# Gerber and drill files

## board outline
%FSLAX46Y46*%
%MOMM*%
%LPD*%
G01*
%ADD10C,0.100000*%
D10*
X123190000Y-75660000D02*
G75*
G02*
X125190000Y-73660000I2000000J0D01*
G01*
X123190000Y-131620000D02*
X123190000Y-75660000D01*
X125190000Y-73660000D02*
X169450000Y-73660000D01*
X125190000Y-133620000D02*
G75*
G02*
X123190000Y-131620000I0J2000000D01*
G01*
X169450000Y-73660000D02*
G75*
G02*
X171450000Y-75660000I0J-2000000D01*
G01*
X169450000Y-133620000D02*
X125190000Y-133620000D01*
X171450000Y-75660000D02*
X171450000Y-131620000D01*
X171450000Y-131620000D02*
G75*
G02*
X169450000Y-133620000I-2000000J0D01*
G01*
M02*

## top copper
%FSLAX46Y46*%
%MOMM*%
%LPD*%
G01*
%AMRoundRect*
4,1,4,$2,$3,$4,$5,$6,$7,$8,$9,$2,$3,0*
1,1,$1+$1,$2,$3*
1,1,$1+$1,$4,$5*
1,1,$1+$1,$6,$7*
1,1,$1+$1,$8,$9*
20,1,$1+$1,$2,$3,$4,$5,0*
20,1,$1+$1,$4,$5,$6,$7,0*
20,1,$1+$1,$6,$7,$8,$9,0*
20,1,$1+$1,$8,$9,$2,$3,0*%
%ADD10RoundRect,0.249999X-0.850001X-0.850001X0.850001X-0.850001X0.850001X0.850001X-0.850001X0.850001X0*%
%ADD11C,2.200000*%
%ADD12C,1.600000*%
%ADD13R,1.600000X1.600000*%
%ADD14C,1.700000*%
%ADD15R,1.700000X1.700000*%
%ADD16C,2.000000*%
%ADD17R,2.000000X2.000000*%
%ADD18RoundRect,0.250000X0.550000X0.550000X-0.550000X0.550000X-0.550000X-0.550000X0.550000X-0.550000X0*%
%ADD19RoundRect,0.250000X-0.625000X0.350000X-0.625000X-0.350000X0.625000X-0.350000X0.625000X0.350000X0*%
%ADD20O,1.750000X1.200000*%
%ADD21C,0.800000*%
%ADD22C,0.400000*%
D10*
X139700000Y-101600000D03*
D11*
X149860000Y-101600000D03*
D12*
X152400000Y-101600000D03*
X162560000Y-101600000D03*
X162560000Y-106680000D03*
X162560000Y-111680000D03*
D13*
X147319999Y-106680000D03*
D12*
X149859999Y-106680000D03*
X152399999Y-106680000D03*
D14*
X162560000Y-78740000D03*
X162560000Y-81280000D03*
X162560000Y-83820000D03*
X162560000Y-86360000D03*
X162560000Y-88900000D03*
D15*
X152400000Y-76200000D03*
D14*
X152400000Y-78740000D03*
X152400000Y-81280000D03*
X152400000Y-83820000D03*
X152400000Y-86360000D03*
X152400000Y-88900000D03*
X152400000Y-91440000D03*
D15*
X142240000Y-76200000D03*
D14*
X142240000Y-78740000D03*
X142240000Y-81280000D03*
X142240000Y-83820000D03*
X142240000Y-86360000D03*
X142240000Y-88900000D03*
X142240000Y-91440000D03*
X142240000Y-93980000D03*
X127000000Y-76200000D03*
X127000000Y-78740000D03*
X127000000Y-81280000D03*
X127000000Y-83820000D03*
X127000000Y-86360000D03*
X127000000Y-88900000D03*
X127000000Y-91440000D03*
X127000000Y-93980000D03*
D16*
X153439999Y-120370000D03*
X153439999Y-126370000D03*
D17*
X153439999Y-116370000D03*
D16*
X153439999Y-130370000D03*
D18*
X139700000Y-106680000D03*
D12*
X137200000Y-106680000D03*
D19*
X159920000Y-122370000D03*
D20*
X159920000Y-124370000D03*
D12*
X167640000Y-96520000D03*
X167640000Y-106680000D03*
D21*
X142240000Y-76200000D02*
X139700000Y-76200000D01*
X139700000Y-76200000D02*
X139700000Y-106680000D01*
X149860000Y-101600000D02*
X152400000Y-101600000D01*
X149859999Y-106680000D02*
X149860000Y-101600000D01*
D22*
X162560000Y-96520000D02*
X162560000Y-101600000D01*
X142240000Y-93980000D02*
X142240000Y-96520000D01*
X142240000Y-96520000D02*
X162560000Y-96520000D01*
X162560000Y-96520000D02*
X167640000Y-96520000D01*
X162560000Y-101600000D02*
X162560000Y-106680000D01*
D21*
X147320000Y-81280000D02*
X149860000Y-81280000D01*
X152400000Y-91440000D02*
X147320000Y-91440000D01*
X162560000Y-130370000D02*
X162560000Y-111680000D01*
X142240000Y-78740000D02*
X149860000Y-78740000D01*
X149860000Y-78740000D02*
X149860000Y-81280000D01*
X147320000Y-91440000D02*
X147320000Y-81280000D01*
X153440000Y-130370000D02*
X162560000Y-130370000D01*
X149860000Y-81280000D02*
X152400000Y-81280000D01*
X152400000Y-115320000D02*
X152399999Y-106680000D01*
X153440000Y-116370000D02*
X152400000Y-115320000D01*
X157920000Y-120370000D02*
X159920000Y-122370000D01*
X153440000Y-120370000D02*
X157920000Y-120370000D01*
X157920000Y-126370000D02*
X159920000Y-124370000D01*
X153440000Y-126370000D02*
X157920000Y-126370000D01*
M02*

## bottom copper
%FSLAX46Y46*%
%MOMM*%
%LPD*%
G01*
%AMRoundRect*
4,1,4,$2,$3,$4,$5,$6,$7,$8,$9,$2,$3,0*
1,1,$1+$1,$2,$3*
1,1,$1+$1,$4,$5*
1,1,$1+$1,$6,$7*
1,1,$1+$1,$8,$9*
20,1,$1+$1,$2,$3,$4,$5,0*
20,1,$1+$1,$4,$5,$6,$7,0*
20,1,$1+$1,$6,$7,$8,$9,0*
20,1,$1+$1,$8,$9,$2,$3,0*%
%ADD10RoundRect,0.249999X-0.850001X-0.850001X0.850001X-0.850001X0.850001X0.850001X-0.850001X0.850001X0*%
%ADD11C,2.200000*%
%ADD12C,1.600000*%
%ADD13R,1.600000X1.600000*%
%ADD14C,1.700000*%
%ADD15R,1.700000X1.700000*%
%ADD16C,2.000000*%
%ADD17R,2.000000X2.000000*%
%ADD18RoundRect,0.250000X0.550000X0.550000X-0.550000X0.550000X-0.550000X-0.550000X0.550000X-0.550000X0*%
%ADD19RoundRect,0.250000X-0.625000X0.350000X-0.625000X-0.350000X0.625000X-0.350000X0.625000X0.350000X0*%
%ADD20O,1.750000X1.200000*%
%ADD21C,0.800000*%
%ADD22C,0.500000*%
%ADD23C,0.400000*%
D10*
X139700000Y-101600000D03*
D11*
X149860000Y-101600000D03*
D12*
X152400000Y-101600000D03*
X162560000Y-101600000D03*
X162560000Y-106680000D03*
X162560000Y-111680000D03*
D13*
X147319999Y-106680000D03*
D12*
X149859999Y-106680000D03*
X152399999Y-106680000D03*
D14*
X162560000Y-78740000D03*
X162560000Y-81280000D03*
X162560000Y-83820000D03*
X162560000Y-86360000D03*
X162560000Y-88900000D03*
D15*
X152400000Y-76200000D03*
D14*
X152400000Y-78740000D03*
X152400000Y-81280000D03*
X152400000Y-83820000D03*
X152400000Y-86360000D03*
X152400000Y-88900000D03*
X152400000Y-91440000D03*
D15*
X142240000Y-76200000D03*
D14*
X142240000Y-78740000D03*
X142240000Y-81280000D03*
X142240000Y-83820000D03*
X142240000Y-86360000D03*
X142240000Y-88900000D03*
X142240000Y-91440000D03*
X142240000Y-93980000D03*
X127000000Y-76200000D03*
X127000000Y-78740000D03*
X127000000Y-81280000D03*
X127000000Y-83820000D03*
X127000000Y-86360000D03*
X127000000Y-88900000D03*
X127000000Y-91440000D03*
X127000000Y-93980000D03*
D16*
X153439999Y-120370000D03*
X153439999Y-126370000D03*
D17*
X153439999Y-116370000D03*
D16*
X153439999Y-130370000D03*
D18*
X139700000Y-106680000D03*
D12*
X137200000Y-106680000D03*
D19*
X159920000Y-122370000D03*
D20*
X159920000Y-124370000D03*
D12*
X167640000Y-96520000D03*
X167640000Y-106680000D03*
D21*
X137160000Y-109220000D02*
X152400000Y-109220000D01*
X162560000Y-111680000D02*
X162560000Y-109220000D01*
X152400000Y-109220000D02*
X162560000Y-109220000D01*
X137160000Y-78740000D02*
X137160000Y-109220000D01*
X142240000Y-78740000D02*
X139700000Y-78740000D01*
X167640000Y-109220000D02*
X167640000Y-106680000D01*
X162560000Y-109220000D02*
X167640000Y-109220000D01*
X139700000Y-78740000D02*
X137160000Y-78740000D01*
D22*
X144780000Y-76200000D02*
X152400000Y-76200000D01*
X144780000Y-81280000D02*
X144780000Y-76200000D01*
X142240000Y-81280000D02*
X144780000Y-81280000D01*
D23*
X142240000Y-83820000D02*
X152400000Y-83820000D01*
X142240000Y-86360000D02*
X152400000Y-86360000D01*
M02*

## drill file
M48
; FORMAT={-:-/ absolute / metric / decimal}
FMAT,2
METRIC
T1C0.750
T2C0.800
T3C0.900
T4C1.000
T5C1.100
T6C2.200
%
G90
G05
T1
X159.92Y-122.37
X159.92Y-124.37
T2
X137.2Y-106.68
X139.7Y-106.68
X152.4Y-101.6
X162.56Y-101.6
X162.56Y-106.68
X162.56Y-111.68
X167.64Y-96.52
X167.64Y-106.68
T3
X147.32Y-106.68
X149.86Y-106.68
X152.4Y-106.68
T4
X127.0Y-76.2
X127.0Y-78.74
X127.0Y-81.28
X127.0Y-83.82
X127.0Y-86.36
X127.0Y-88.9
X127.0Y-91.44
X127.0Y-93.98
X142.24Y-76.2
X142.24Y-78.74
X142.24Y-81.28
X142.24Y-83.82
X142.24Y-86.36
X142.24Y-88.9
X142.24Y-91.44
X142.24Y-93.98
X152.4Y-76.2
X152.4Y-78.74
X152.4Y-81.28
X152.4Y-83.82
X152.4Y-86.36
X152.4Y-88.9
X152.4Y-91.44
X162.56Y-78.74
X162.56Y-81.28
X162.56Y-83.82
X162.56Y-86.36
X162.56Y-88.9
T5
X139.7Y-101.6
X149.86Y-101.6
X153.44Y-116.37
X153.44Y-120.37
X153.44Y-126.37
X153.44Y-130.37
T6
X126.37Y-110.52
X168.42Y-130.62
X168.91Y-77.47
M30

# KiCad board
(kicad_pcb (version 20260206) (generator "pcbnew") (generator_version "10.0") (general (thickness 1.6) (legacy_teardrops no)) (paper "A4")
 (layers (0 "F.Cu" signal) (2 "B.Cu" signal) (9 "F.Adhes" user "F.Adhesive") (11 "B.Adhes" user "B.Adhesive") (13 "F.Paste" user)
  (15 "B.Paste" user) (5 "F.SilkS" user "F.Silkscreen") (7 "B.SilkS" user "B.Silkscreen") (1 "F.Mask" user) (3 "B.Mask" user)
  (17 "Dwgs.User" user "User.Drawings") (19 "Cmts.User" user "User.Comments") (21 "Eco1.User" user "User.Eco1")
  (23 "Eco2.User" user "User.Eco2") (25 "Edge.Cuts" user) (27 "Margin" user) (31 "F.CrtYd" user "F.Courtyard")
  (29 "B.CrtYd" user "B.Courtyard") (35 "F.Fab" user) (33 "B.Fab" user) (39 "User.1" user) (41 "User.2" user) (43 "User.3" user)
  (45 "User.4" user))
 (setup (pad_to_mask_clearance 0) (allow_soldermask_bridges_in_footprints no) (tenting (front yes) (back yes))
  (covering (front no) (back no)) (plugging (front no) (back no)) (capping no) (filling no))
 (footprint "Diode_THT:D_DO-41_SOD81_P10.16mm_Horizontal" (layer "F.Cu") (at 139.7 101.6)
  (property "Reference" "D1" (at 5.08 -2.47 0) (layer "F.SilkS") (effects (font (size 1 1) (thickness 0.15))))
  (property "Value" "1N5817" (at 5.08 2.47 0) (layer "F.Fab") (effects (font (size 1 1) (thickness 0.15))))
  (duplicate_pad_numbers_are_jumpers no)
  (pad "1" thru_hole roundrect (at 0 0) (size 2.2 2.2) (drill 1.1) (layers "*.Cu" "*.Mask") (remove_unused_layers no)
   (roundrect_rratio 0.113636) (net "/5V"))
  (pad "2" thru_hole circle (at 10.16 0) (size 2.2 2.2) (drill 1.1) (layers "*.Cu" "*.Mask") (remove_unused_layers no) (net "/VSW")))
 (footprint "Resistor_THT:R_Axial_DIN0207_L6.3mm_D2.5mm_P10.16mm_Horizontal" (layer "F.Cu") (at 152.4 101.6)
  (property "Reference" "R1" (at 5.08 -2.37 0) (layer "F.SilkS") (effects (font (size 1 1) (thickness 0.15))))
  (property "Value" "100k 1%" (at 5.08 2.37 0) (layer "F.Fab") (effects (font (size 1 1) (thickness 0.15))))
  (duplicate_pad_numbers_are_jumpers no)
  (pad "1" thru_hole circle (at 0 0) (size 1.6 1.6) (drill 0.8) (layers "*.Cu" "*.Mask") (remove_unused_layers no) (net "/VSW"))
  (pad "2" thru_hole circle (at 10.16 0) (size 1.6 1.6) (drill 0.8) (layers "*.Cu" "*.Mask") (remove_unused_layers no) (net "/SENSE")))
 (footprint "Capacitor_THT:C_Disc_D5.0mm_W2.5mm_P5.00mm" (layer "F.Cu") (at 162.56 106.68 -90)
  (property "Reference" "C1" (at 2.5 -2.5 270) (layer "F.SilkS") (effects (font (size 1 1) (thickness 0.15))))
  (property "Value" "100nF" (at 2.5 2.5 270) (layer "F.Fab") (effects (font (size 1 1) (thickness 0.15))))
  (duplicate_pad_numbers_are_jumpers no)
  (pad "1" thru_hole circle (at 0 0 270) (size 1.6 1.6) (drill 0.8) (layers "*.Cu" "*.Mask") (remove_unused_layers no) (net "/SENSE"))
  (pad "2" thru_hole circle (at 5 0 270) (size 1.6 1.6) (drill 0.8) (layers "*.Cu" "*.Mask") (remove_unused_layers no) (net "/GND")))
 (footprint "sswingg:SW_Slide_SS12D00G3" (layer "F.Cu") (at 149.859999 106.68)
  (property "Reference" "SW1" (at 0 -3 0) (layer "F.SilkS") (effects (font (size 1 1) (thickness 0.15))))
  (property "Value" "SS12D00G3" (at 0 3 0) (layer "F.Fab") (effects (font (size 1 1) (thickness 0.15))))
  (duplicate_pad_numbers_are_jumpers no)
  (pad "1" thru_hole rect (at -2.54 0) (size 1.6 1.6) (drill 0.9) (layers "*.Cu" "*.Mask") (remove_unused_layers no)
   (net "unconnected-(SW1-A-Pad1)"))
  (pad "2" thru_hole circle (at 0 0) (size 1.6 1.6) (drill 0.9) (layers "*.Cu" "*.Mask") (remove_unused_layers no) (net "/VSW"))
  (pad "3" thru_hole circle (at 2.54 0) (size 1.6 1.6) (drill 0.9) (layers "*.Cu" "*.Mask") (remove_unused_layers no) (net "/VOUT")))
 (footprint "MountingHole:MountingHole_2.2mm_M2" (layer "F.Cu") (at 168.42 130.62)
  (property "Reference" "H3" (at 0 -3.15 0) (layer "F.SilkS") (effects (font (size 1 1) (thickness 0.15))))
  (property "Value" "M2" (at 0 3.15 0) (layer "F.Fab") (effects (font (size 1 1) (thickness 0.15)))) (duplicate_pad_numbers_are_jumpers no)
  (pad "" np_thru_hole circle (at 0 0) (size 2.2 2.2) (drill 2.2) (layers "*.Cu" "*.Mask")))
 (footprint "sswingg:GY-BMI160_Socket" (layer "F.Cu") (at 152.4 76.2)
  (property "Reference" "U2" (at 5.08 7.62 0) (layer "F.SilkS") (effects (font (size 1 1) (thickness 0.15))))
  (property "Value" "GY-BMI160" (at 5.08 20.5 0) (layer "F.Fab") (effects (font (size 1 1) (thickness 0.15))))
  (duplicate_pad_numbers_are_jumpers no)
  (pad "" thru_hole circle (at 10.16 2.54) (size 1.7 1.7) (drill 1) (layers "*.Cu" "*.Mask") (remove_unused_layers no))
  (pad "" thru_hole circle (at 10.16 5.08) (size 1.7 1.7) (drill 1) (layers "*.Cu" "*.Mask") (remove_unused_layers no))
  (pad "" thru_hole circle (at 10.16 7.62) (size 1.7 1.7) (drill 1) (layers "*.Cu" "*.Mask") (remove_unused_layers no))
  (pad "" thru_hole circle (at 10.16 10.16) (size 1.7 1.7) (drill 1) (layers "*.Cu" "*.Mask") (remove_unused_layers no))
  (pad "" thru_hole circle (at 10.16 12.7) (size 1.7 1.7) (drill 1) (layers "*.Cu" "*.Mask") (remove_unused_layers no))
  (pad "1" thru_hole rect (at 0 0) (size 1.7 1.7) (drill 1) (layers "*.Cu" "*.Mask") (remove_unused_layers no) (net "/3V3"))
  (pad "2" thru_hole circle (at 0 2.54) (size 1.7 1.7) (drill 1) (layers "*.Cu" "*.Mask") (remove_unused_layers no)
   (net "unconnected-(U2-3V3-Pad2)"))
  (pad "3" thru_hole circle (at 0 5.08) (size 1.7 1.7) (drill 1) (layers "*.Cu" "*.Mask") (remove_unused_layers no) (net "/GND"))
  (pad "4" thru_hole circle (at 0 7.62) (size 1.7 1.7) (drill 1) (layers "*.Cu" "*.Mask") (remove_unused_layers no) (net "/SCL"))
  (pad "5" thru_hole circle (at 0 10.16) (size 1.7 1.7) (drill 1) (layers "*.Cu" "*.Mask") (remove_unused_layers no) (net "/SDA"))
  (pad "6" thru_hole circle (at 0 12.7) (size 1.7 1.7) (drill 1) (layers "*.Cu" "*.Mask") (remove_unused_layers no)
   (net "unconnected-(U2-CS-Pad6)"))
  (pad "7" thru_hole circle (at 0 15.24) (size 1.7 1.7) (drill 1) (layers "*.Cu" "*.Mask") (remove_unused_layers no) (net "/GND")))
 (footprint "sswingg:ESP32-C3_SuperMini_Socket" (layer "F.Cu") (at 142.24 76.2)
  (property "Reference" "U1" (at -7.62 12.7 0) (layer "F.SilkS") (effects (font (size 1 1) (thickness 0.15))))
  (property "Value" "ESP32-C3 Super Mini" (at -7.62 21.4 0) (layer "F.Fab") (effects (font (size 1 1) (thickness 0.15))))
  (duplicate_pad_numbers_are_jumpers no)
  (pad "1" thru_hole rect (at 0 0) (size 1.7 1.7) (drill 1) (layers "*.Cu" "*.Mask") (remove_unused_layers no) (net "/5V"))
  (pad "2" thru_hole circle (at 0 2.54) (size 1.7 1.7) (drill 1) (layers "*.Cu" "*.Mask") (remove_unused_layers no) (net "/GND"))
  (pad "3" thru_hole circle (at 0 5.08) (size 1.7 1.7) (drill 1) (layers "*.Cu" "*.Mask") (remove_unused_layers no) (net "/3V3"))
  (pad "4" thru_hole circle (at 0 7.62) (size 1.7 1.7) (drill 1) (layers "*.Cu" "*.Mask") (remove_unused_layers no) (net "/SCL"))
  (pad "5" thru_hole circle (at 0 10.16) (size 1.7 1.7) (drill 1) (layers "*.Cu" "*.Mask") (remove_unused_layers no) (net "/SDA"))
  (pad "6" thru_hole circle (at 0 12.7) (size 1.7 1.7) (drill 1) (layers "*.Cu" "*.Mask") (remove_unused_layers no)
   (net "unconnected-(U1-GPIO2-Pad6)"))
  (pad "7" thru_hole circle (at 0 15.24) (size 1.7 1.7) (drill 1) (layers "*.Cu" "*.Mask") (remove_unused_layers no)
   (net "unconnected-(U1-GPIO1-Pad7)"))
  (pad "8" thru_hole circle (at 0 17.78) (size 1.7 1.7) (drill 1) (layers "*.Cu" "*.Mask") (remove_unused_layers no) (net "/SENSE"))
  (pad "9" thru_hole circle (at -15.24 0) (size 1.7 1.7) (drill 1) (layers "*.Cu" "*.Mask") (remove_unused_layers no)
   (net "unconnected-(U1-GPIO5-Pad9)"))
  (pad "10" thru_hole circle (at -15.24 2.54) (size 1.7 1.7) (drill 1) (layers "*.Cu" "*.Mask") (remove_unused_layers no)
   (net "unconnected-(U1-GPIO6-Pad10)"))
  (pad "11" thru_hole circle (at -15.24 5.08) (size 1.7 1.7) (drill 1) (layers "*.Cu" "*.Mask") (remove_unused_layers no)
   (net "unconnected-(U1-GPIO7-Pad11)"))
  (pad "12" thru_hole circle (at -15.24 7.62) (size 1.7 1.7) (drill 1) (layers "*.Cu" "*.Mask") (remove_unused_layers no)
   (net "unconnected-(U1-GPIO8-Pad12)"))
  (pad "13" thru_hole circle (at -15.24 10.16) (size 1.7 1.7) (drill 1) (layers "*.Cu" "*.Mask") (remove_unused_layers no)
   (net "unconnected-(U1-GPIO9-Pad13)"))
  (pad "14" thru_hole circle (at -15.24 12.7) (size 1.7 1.7) (drill 1) (layers "*.Cu" "*.Mask") (remove_unused_layers no)
   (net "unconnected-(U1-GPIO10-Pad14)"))
  (pad "15" thru_hole circle (at -15.24 15.24) (size 1.7 1.7) (drill 1) (layers "*.Cu" "*.Mask") (remove_unused_layers no)
   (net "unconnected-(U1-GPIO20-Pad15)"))
  (pad "16" thru_hole circle (at -15.24 17.78) (size 1.7 1.7) (drill 1) (layers "*.Cu" "*.Mask") (remove_unused_layers no)
   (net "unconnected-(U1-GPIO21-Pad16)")))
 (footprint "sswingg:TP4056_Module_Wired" (layer "F.Cu") (at 123.189999 114.62)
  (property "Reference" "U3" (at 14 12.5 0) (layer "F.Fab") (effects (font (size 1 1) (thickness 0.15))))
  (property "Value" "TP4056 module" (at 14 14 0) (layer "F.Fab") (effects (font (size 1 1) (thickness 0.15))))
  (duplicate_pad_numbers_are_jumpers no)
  (pad "3" thru_hole circle (at 30.25 5.75) (size 2 2) (drill 1.1) (layers "*.Cu" "*.Mask") (remove_unused_layers no) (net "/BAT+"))
  (pad "4" thru_hole circle (at 30.25 11.75) (size 2 2) (drill 1.1) (layers "*.Cu" "*.Mask") (remove_unused_layers no) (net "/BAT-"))
  (pad "5" thru_hole rect (at 30.25 1.75) (size 2 2) (drill 1.1) (layers "*.Cu" "*.Mask") (remove_unused_layers no) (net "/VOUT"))
  (pad "6" thru_hole circle (at 30.25 15.75) (size 2 2) (drill 1.1) (layers "*.Cu" "*.Mask") (remove_unused_layers no) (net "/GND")))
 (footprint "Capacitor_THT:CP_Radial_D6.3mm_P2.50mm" (layer "F.Cu") (at 139.7 106.68 180)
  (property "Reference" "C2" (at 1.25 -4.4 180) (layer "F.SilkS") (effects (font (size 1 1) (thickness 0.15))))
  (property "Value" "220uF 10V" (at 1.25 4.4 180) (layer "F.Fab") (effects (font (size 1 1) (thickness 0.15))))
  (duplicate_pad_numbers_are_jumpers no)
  (pad "1" thru_hole roundrect (at 0 0 180) (size 1.6 1.6) (drill 0.8) (layers "*.Cu" "*.Mask") (remove_unused_layers no)
   (roundrect_rratio 0.15625) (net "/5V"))
  (pad "2" thru_hole circle (at 2.5 0 180) (size 1.6 1.6) (drill 0.8) (layers "*.Cu" "*.Mask") (remove_unused_layers no) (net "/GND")))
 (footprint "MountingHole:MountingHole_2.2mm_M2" (layer "F.Cu") (at 168.91 77.47)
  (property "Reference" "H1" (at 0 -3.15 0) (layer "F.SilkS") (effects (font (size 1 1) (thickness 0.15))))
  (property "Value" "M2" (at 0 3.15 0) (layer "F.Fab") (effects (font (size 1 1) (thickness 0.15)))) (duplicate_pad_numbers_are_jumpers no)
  (pad "" np_thru_hole circle (at 0 0) (size 2.2 2.2) (drill 2.2) (layers "*.Cu" "*.Mask")))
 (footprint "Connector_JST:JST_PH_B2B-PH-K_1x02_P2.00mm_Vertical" (layer "F.Cu") (at 159.92 122.37 -90)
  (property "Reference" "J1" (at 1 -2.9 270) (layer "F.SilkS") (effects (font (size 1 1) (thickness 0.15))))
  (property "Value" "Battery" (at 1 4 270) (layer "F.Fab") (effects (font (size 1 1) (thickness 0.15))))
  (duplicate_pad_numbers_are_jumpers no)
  (pad "1" thru_hole roundrect (at 0 0 270) (size 1.2 1.75) (drill 0.75) (layers "*.Cu" "*.Mask") (remove_unused_layers no)
   (roundrect_rratio 0.208333) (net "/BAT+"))
  (pad "2" thru_hole oval (at 2 0 270) (size 1.2 1.75) (drill 0.75) (layers "*.Cu" "*.Mask") (remove_unused_layers no) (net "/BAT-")))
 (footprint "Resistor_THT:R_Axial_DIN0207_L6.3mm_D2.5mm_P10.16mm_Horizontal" (layer "F.Cu") (at 167.64 96.52 -90)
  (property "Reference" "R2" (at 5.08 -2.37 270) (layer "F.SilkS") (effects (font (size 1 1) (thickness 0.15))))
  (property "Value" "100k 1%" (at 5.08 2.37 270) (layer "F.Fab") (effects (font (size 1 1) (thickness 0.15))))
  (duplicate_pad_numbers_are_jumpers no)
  (pad "1" thru_hole circle (at 0 0 270) (size 1.6 1.6) (drill 0.8) (layers "*.Cu" "*.Mask") (remove_unused_layers no) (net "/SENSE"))
  (pad "2" thru_hole circle (at 10.16 0 270) (size 1.6 1.6) (drill 0.8) (layers "*.Cu" "*.Mask") (remove_unused_layers no) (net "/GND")))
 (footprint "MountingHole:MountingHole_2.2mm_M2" (layer "F.Cu") (at 126.37 110.52)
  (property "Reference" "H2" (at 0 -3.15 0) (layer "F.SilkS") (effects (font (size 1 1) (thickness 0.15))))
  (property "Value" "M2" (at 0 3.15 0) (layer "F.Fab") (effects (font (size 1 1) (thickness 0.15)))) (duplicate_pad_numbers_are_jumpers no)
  (pad "" np_thru_hole circle (at 0 0) (size 2.2 2.2) (drill 2.2) (layers "*.Cu" "*.Mask")))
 (gr_arc (start 123.19 75.66) (mid 123.775786 74.245786) (end 125.19 73.66) (stroke (width 0.1) (type default)) (layer "Edge.Cuts"))
 (gr_line (start 123.19 131.62) (end 123.19 75.66) (stroke (width 0.1) (type default)) (layer "Edge.Cuts"))
 (gr_line (start 125.19 73.66) (end 169.45 73.66) (stroke (width 0.1) (type default)) (layer "Edge.Cuts"))
 (gr_arc (start 125.19 133.62) (mid 123.775786 133.034213) (end 123.19 131.62) (stroke (width 0.1) (type default)) (layer "Edge.Cuts"))
 (gr_arc (start 169.45 73.66) (mid 170.864213 74.245786) (end 171.45 75.66) (stroke (width 0.1) (type default)) (layer "Edge.Cuts"))
 (gr_line (start 169.45 133.62) (end 125.19 133.62) (stroke (width 0.1) (type default)) (layer "Edge.Cuts"))
 (gr_line (start 171.45 75.66) (end 171.45 131.62) (stroke (width 0.1) (type default)) (layer "Edge.Cuts"))
 (gr_arc (start 171.45 131.62) (mid 170.864213 133.034213) (end 169.45 133.62) (stroke (width 0.1) (type default)) (layer "Edge.Cuts"))
 (segment (start 142.24 76.2) (end 139.7 76.2) (width 0.8) (layer "F.Cu") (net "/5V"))
 (segment (start 139.7 76.2) (end 139.7 106.68) (width 0.8) (layer "F.Cu") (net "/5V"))
 (segment (start 149.86 101.6) (end 152.4 101.6) (width 0.8) (layer "F.Cu") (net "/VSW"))
 (segment (start 149.859999 106.68) (end 149.86 101.6) (width 0.8) (layer "F.Cu") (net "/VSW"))
 (segment (start 162.56 96.52) (end 162.56 101.6) (width 0.4) (layer "F.Cu") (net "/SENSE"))
 (segment (start 142.24 93.98) (end 142.24 96.52) (width 0.4) (layer "F.Cu") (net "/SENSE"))
 (segment (start 142.24 96.52) (end 162.56 96.52) (width 0.4) (layer "F.Cu") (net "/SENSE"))
 (segment (start 162.56 96.52) (end 167.64 96.52) (width 0.4) (layer "F.Cu") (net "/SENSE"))
 (segment (start 162.56 101.6) (end 162.56 106.68) (width 0.4) (layer "F.Cu") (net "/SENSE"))
 (segment (start 147.32 81.28) (end 149.86 81.28) (width 0.8) (layer "F.Cu") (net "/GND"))
 (segment (start 152.4 91.44) (end 147.32 91.44) (width 0.8) (layer "F.Cu") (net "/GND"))
 (segment (start 162.56 130.37) (end 162.56 111.68) (width 0.8) (layer "F.Cu") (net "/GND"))
 (segment (start 142.24 78.74) (end 149.86 78.74) (width 0.8) (layer "F.Cu") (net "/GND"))
 (segment (start 149.86 78.74) (end 149.86 81.28) (width 0.8) (layer "F.Cu") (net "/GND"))
 (segment (start 147.32 91.44) (end 147.32 81.28) (width 0.8) (layer "F.Cu") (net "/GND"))
 (segment (start 153.44 130.37) (end 162.56 130.37) (width 0.8) (layer "F.Cu") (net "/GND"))
 (segment (start 149.86 81.28) (end 152.4 81.28) (width 0.8) (layer "F.Cu") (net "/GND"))
 (segment (start 137.16 109.22) (end 152.4 109.22) (width 0.8) (layer "B.Cu") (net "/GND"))
 (segment (start 162.56 111.68) (end 162.56 109.22) (width 0.8) (layer "B.Cu") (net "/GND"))
 (segment (start 152.4 109.22) (end 162.56 109.22) (width 0.8) (layer "B.Cu") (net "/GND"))
 (segment (start 137.16 78.74) (end 137.16 109.22) (width 0.8) (layer "B.Cu") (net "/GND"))
 (segment (start 142.24 78.74) (end 139.7 78.74) (width 0.8) (layer "B.Cu") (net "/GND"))
 (segment (start 167.64 109.22) (end 167.64 106.68) (width 0.8) (layer "B.Cu") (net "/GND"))
 (segment (start 162.56 109.22) (end 167.64 109.22) (width 0.8) (layer "B.Cu") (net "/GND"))
 (segment (start 139.7 78.74) (end 137.16 78.74) (width 0.8) (layer "B.Cu") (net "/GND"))
 (segment (start 152.4 115.32) (end 152.399999 106.68) (width 0.8) (layer "F.Cu") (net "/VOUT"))
 (segment (start 153.44 116.37) (end 152.4 115.32) (width 0.8) (layer "F.Cu") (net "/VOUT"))
 (segment (start 144.78 76.2) (end 152.4 76.2) (width 0.5) (layer "B.Cu") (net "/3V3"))
 (segment (start 144.78 81.28) (end 144.78 76.2) (width 0.5) (layer "B.Cu") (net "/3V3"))
 (segment (start 142.24 81.28) (end 144.78 81.28) (width 0.5) (layer "B.Cu") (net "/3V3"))
 (segment (start 142.24 83.82) (end 152.4 83.82) (width 0.4) (layer "B.Cu") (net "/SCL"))
 (segment (start 142.24 86.36) (end 152.4 86.36) (width 0.4) (layer "B.Cu") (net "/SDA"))
 (segment (start 157.92 120.37) (end 159.92 122.37) (width 0.8) (layer "F.Cu") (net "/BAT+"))
 (segment (start 153.44 120.37) (end 157.92 120.37) (width 0.8) (layer "F.Cu") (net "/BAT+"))
 (segment (start 157.92 126.37) (end 159.92 124.37) (width 0.8) (layer "F.Cu") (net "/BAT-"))
 (segment (start 153.44 126.37) (end 157.92 126.37) (width 0.8) (layer "F.Cu") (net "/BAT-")))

